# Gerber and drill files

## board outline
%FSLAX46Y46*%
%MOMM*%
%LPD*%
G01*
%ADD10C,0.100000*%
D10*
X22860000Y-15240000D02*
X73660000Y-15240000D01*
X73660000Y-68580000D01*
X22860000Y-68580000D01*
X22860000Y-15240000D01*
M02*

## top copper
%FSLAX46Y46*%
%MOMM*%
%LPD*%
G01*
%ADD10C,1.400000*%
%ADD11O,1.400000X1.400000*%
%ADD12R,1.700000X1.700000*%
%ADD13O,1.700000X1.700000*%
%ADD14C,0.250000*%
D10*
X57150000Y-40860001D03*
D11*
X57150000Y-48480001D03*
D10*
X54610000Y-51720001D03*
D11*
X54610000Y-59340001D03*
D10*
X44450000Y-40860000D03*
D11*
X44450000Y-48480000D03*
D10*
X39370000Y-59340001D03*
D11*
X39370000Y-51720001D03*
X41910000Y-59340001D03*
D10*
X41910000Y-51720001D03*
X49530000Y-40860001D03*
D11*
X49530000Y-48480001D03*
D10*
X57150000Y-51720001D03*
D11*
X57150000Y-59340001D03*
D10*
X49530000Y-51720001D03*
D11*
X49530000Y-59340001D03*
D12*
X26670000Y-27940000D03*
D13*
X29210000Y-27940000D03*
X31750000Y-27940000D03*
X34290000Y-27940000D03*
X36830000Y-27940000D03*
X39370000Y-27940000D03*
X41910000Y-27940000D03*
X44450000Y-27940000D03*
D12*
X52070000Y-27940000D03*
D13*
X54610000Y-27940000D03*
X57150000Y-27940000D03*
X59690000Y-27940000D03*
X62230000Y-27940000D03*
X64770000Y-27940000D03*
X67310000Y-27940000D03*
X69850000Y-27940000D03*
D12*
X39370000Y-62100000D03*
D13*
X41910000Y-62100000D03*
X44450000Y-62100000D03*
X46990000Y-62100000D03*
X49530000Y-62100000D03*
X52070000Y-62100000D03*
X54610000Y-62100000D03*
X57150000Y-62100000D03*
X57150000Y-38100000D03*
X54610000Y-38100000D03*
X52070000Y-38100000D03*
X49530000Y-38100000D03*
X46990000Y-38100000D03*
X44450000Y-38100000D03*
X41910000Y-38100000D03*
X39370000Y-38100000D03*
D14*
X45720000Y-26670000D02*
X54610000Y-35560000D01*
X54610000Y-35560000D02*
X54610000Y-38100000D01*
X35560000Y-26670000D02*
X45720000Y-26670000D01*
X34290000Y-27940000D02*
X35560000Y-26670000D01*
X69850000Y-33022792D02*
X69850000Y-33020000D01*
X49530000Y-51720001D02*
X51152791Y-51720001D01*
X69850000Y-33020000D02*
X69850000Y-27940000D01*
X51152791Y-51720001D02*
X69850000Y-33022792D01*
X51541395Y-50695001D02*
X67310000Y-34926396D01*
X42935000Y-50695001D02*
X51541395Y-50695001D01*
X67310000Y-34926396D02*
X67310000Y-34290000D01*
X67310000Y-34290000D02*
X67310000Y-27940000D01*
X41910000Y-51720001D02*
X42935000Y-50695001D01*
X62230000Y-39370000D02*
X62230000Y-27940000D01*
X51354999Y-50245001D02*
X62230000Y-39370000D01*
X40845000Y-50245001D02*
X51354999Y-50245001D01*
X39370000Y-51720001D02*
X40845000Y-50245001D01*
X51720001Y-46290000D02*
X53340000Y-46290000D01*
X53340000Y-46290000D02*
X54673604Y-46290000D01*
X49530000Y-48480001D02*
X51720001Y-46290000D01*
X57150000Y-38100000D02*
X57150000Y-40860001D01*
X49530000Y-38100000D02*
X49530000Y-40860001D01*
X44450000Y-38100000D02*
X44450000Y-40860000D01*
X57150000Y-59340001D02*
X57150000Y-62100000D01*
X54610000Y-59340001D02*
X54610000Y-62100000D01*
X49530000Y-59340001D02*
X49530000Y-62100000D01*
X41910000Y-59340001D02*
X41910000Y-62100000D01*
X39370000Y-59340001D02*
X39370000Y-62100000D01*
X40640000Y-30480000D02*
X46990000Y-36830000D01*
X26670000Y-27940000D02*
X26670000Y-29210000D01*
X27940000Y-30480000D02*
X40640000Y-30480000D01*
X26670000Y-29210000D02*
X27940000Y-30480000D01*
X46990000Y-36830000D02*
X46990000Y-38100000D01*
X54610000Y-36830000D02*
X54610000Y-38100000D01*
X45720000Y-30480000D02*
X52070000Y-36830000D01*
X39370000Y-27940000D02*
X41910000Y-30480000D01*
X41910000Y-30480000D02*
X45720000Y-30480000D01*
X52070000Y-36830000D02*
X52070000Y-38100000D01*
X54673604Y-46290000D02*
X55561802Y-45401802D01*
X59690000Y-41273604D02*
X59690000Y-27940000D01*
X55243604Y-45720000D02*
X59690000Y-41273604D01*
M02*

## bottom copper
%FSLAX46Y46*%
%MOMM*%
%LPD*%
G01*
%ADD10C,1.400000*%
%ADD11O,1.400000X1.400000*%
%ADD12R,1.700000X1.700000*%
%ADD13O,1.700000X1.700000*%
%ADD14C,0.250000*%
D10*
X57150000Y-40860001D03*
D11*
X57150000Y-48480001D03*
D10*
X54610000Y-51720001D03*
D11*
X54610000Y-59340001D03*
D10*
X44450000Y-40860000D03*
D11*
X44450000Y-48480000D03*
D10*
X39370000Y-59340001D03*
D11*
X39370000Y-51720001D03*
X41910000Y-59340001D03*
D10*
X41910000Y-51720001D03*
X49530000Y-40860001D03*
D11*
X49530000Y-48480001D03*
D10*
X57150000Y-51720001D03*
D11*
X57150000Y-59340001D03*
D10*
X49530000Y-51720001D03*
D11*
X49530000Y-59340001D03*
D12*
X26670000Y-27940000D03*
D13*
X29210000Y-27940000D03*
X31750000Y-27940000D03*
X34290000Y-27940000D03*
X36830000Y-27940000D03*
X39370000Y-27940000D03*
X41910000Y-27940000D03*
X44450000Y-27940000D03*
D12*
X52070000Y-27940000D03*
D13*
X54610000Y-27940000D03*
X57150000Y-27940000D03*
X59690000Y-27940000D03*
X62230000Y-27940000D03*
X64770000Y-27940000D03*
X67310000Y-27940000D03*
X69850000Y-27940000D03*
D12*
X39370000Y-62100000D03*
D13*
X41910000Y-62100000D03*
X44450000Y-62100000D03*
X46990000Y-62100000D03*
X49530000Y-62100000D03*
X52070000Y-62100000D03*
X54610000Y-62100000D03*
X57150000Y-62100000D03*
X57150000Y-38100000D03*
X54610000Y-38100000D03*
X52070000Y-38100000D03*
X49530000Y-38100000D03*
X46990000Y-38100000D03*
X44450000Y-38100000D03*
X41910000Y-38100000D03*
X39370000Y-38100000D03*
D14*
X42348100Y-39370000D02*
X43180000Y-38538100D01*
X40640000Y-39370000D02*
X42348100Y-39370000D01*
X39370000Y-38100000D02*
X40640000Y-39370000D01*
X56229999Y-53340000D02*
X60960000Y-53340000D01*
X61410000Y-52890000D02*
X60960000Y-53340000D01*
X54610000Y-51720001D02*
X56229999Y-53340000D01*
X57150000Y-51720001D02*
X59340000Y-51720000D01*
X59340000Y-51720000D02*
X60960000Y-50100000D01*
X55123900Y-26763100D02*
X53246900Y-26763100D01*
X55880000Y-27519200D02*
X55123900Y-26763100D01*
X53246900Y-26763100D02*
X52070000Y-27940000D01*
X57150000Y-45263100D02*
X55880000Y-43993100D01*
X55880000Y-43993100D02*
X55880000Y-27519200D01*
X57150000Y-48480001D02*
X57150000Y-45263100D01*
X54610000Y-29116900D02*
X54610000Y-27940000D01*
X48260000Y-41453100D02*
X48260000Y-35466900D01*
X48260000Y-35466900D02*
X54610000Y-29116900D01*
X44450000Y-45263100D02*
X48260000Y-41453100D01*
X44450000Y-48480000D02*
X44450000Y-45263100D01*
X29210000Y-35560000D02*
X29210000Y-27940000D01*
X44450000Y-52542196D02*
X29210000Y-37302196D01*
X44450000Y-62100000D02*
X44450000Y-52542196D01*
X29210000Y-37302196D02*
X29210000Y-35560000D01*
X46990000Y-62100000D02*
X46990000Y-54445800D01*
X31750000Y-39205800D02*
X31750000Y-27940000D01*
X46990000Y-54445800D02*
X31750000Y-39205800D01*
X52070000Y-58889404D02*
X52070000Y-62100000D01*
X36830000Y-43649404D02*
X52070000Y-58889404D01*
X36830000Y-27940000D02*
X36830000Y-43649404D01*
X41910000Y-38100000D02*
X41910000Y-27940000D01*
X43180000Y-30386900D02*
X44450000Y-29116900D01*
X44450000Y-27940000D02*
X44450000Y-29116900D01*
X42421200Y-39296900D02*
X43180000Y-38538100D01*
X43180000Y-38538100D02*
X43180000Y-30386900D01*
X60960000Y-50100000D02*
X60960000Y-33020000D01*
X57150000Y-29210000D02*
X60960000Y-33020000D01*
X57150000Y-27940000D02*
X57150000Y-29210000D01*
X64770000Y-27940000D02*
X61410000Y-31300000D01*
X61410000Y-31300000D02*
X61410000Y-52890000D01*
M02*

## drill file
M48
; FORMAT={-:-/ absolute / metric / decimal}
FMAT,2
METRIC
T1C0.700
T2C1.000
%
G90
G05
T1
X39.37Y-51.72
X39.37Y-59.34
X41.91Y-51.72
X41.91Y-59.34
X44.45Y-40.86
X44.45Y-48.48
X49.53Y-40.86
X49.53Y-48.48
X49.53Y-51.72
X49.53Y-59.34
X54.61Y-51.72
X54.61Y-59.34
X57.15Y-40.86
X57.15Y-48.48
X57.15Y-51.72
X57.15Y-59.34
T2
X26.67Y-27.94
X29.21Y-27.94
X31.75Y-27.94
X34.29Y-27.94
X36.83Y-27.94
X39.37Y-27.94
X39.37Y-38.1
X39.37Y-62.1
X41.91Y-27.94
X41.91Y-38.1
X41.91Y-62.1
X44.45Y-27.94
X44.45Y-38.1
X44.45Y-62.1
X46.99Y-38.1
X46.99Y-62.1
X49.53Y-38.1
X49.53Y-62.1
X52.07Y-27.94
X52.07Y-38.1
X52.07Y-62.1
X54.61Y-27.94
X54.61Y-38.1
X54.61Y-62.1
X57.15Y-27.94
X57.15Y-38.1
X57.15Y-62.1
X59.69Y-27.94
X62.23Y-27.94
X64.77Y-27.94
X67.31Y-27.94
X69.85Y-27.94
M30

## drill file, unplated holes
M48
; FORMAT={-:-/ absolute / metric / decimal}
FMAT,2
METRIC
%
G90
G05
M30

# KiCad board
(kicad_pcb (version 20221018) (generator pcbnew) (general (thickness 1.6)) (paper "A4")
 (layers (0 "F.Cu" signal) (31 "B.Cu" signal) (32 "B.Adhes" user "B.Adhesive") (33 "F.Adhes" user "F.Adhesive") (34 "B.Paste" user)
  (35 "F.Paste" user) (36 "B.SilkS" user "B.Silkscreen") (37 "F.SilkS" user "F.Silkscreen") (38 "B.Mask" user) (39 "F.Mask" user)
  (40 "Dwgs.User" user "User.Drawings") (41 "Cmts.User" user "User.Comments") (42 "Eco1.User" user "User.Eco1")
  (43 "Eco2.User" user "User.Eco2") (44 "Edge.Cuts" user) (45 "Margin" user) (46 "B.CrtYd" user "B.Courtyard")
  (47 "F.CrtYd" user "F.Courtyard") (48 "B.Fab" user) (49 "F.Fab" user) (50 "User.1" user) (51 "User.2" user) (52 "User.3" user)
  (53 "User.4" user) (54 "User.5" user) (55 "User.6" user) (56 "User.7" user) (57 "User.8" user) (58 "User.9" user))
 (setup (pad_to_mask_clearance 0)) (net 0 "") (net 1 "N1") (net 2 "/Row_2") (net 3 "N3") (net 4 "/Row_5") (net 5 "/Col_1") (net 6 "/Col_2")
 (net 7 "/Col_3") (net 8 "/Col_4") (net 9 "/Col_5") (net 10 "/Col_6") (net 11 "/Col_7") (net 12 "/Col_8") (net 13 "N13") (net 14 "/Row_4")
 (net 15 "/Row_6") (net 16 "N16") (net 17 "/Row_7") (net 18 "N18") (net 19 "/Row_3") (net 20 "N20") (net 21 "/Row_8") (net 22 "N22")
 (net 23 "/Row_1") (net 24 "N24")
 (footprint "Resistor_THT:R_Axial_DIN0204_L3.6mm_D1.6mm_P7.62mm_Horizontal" (layer "F.Cu") (at 44.45 40.86 -90)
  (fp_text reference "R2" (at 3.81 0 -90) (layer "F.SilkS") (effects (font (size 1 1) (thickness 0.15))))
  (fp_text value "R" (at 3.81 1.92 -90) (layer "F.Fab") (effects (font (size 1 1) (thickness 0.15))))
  (pad "1" thru_hole circle (at 0 0 270) (size 1.4 1.4) (drill 0.7) (layers "*.Cu" "*.Mask") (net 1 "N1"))
  (pad "2" thru_hole oval (at 7.62 0 270) (size 1.4 1.4) (drill 0.7) (layers "*.Cu" "*.Mask") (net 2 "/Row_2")))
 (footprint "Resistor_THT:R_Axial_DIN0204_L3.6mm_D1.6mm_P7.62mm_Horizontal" (layer "F.Cu") (at 39.37 59.340001 90)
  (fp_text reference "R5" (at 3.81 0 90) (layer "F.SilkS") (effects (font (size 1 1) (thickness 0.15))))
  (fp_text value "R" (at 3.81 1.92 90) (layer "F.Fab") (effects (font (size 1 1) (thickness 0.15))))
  (pad "1" thru_hole circle (at 0 0 90) (size 1.4 1.4) (drill 0.7) (layers "*.Cu" "*.Mask") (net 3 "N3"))
  (pad "2" thru_hole oval (at 7.62 0 90) (size 1.4 1.4) (drill 0.7) (layers "*.Cu" "*.Mask") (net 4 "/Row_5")))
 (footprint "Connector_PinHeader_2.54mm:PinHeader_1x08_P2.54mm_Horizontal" (layer "F.Cu") (at 26.67 27.94 90)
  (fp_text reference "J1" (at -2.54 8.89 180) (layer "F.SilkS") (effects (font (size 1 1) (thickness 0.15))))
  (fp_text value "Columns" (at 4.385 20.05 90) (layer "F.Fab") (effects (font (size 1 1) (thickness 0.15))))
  (pad "1" thru_hole rect (at 0 0 90) (size 1.7 1.7) (drill 1) (layers "*.Cu" "*.Mask") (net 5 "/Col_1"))
  (pad "2" thru_hole oval (at 0 2.54 90) (size 1.7 1.7) (drill 1) (layers "*.Cu" "*.Mask") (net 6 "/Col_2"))
  (pad "3" thru_hole oval (at 0 5.08 90) (size 1.7 1.7) (drill 1) (layers "*.Cu" "*.Mask") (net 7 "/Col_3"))
  (pad "4" thru_hole oval (at 0 7.62 90) (size 1.7 1.7) (drill 1) (layers "*.Cu" "*.Mask") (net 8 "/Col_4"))
  (pad "5" thru_hole oval (at 0 10.16 90) (size 1.7 1.7) (drill 1) (layers "*.Cu" "*.Mask") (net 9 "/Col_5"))
  (pad "6" thru_hole oval (at 0 12.7 90) (size 1.7 1.7) (drill 1) (layers "*.Cu" "*.Mask") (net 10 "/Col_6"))
  (pad "7" thru_hole oval (at 0 15.24 90) (size 1.7 1.7) (drill 1) (layers "*.Cu" "*.Mask") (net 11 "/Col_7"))
  (pad "8" thru_hole oval (at 0 17.78 90) (size 1.7 1.7) (drill 1) (layers "*.Cu" "*.Mask") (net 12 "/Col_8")))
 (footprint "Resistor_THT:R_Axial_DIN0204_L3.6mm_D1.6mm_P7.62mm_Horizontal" (layer "F.Cu") (at 49.53 40.860001 -90)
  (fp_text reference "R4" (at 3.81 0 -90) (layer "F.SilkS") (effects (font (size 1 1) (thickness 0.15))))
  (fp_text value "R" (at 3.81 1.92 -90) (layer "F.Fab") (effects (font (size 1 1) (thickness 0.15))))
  (pad "1" thru_hole circle (at 0 0 270) (size 1.4 1.4) (drill 0.7) (layers "*.Cu" "*.Mask") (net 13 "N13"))
  (pad "2" thru_hole oval (at 7.62 0 270) (size 1.4 1.4) (drill 0.7) (layers "*.Cu" "*.Mask") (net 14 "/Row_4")))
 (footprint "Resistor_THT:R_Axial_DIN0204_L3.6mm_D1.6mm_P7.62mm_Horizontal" (layer "F.Cu") (at 54.61 51.720001 -90)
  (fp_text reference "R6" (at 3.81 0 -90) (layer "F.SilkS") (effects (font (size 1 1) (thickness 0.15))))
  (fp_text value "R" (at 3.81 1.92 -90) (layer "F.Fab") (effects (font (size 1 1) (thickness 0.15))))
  (pad "1" thru_hole circle (at 0 0 270) (size 1.4 1.4) (drill 0.7) (layers "*.Cu" "*.Mask") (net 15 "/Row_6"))
  (pad "2" thru_hole oval (at 7.62 0 270) (size 1.4 1.4) (drill 0.7) (layers "*.Cu" "*.Mask") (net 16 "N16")))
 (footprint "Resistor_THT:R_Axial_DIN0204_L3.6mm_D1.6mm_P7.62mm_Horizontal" (layer "F.Cu") (at 41.91 51.720001 -90)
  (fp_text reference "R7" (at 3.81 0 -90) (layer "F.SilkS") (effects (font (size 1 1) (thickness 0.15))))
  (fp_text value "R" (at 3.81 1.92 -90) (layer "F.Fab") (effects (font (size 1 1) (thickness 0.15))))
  (pad "1" thru_hole circle (at 0 0 270) (size 1.4 1.4) (drill 0.7) (layers "*.Cu" "*.Mask") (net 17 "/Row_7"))
  (pad "2" thru_hole oval (at 7.62 0 270) (size 1.4 1.4) (drill 0.7) (layers "*.Cu" "*.Mask") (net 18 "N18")))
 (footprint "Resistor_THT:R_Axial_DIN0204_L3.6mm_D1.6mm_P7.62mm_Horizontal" (layer "F.Cu") (at 57.15 51.720001 -90)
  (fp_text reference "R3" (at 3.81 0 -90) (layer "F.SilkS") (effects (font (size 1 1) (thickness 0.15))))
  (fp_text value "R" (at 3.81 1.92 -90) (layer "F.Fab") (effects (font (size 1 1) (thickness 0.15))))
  (pad "1" thru_hole circle (at 0 0 270) (size 1.4 1.4) (drill 0.7) (layers "*.Cu" "*.Mask") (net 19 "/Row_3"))
  (pad "2" thru_hole oval (at 7.62 0 270) (size 1.4 1.4) (drill 0.7) (layers "*.Cu" "*.Mask") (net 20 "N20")))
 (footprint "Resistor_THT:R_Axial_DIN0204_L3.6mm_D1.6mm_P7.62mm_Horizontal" (layer "F.Cu") (at 49.53 51.720001 -90)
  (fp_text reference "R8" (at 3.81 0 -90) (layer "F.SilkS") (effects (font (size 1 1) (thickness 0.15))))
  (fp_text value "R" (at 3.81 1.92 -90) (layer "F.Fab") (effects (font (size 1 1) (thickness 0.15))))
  (pad "1" thru_hole circle (at 0 0 270) (size 1.4 1.4) (drill 0.7) (layers "*.Cu" "*.Mask") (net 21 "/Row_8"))
  (pad "2" thru_hole oval (at 7.62 0 270) (size 1.4 1.4) (drill 0.7) (layers "*.Cu" "*.Mask") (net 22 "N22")))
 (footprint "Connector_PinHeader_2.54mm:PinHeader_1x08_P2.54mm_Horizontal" (layer "F.Cu") (at 52.07 27.94 90)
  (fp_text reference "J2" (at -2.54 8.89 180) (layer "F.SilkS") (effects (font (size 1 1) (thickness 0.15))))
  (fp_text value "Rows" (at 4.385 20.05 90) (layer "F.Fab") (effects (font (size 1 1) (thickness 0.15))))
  (pad "1" thru_hole rect (at 0 0 90) (size 1.7 1.7) (drill 1) (layers "*.Cu" "*.Mask") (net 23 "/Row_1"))
  (pad "2" thru_hole oval (at 0 2.54 90) (size 1.7 1.7) (drill 1) (layers "*.Cu" "*.Mask") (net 2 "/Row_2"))
  (pad "3" thru_hole oval (at 0 5.08 90) (size 1.7 1.7) (drill 1) (layers "*.Cu" "*.Mask") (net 19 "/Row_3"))
  (pad "4" thru_hole oval (at 0 7.62 90) (size 1.7 1.7) (drill 1) (layers "*.Cu" "*.Mask") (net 14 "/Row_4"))
  (pad "5" thru_hole oval (at 0 10.16 90) (size 1.7 1.7) (drill 1) (layers "*.Cu" "*.Mask") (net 4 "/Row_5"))
  (pad "6" thru_hole oval (at 0 12.7 90) (size 1.7 1.7) (drill 1) (layers "*.Cu" "*.Mask") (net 15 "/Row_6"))
  (pad "7" thru_hole oval (at 0 15.24 90) (size 1.7 1.7) (drill 1) (layers "*.Cu" "*.Mask") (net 17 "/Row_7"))
  (pad "8" thru_hole oval (at 0 17.78 90) (size 1.7 1.7) (drill 1) (layers "*.Cu" "*.Mask") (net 21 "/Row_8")))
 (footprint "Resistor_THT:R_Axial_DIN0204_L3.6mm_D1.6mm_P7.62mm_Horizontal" (layer "F.Cu") (at 57.15 40.860001 -90)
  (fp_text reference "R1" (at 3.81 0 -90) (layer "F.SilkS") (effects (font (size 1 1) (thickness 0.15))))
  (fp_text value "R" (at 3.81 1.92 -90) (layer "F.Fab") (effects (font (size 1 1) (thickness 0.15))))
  (pad "1" thru_hole circle (at 0 0 270) (size 1.4 1.4) (drill 0.7) (layers "*.Cu" "*.Mask") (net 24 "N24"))
  (pad "2" thru_hole oval (at 7.62 0 270) (size 1.4 1.4) (drill 0.7) (layers "*.Cu" "*.Mask") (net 23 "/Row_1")))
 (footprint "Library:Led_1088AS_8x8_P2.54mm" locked (layer "F.Cu") (at 48.26 50.1)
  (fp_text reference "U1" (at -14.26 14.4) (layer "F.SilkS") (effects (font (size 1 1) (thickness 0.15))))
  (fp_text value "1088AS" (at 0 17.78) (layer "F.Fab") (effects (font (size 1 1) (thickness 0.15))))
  (pad "1" thru_hole rect locked (at -8.89 12) (size 1.7 1.7) (drill 1) (layers "*.Cu" "*.Mask") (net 3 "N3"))
  (pad "2" thru_hole oval locked (at -6.35 12) (size 1.7 1.7) (drill 1) (layers "*.Cu" "*.Mask") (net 18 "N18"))
  (pad "3" thru_hole oval locked (at -3.81 12) (size 1.7 1.7) (drill 1) (layers "*.Cu" "*.Mask") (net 6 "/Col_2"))
  (pad "4" thru_hole oval locked (at -1.27 12) (size 1.7 1.7) (drill 1) (layers "*.Cu" "*.Mask") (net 7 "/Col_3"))
  (pad "5" thru_hole oval locked (at 1.27 12) (size 1.7 1.7) (drill 1) (layers "*.Cu" "*.Mask") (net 22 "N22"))
  (pad "6" thru_hole oval locked (at 3.81 12) (size 1.7 1.7) (drill 1) (layers "*.Cu" "*.Mask") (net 9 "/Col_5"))
  (pad "7" thru_hole oval locked (at 6.35 12) (size 1.7 1.7) (drill 1) (layers "*.Cu" "*.Mask") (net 16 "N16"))
  (pad "8" thru_hole oval locked (at 8.89 12) (size 1.7 1.7) (drill 1) (layers "*.Cu" "*.Mask") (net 20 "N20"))
  (pad "9" thru_hole oval locked (at 8.89 -12) (size 1.7 1.7) (drill 1) (layers "*.Cu" "*.Mask") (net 24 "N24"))
  (pad "10" thru_hole oval locked (at 6.35 -12) (size 1.7 1.7) (drill 1) (layers "*.Cu" "*.Mask") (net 8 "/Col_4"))
  (pad "11" thru_hole oval locked (at 3.81 -12) (size 1.7 1.7) (drill 1) (layers "*.Cu" "*.Mask") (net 10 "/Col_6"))
  (pad "12" thru_hole oval locked (at 1.27 -12) (size 1.7 1.7) (drill 1) (layers "*.Cu" "*.Mask") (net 13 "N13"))
  (pad "13" thru_hole oval locked (at -1.27 -12) (size 1.7 1.7) (drill 1) (layers "*.Cu" "*.Mask") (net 5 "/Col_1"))
  (pad "14" thru_hole oval locked (at -3.81 -12) (size 1.7 1.7) (drill 1) (layers "*.Cu" "*.Mask") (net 1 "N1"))
  (pad "15" thru_hole oval locked (at -6.35 -12) (size 1.7 1.7) (drill 1) (layers "*.Cu" "*.Mask") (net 11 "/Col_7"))
  (pad "16" thru_hole oval locked (at -8.89 -12) (size 1.7 1.7) (drill 1) (layers "*.Cu" "*.Mask") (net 12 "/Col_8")))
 (gr_rect (start 22.86 15.24) (end 73.66 68.58) (stroke (width 0.1) (type default)) (fill none) (layer "Edge.Cuts"))
 (segment (start 40.64 30.48) (end 46.99 36.83) (width 0.25) (layer "F.Cu") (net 5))
 (segment (start 26.67 27.94) (end 26.67 29.21) (width 0.25) (layer "F.Cu") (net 5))
 (segment (start 27.94 30.48) (end 40.64 30.48) (width 0.25) (layer "F.Cu") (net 5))
 (segment (start 26.67 29.21) (end 27.94 30.48) (width 0.25) (layer "F.Cu") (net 5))
 (segment (start 46.99 36.83) (end 46.99 38.1) (width 0.25) (layer "F.Cu") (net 5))
 (segment (start 29.21 35.56) (end 29.21 27.94) (width 0.25) (layer "B.Cu") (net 6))
 (segment (start 44.45 52.542196) (end 29.21 37.302196) (width 0.25) (layer "B.Cu") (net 6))
 (segment (start 44.45 62.1) (end 44.45 52.542196) (width 0.25) (layer "B.Cu") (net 6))
 (segment (start 29.21 37.302196) (end 29.21 35.56) (width 0.25) (layer "B.Cu") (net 6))
 (segment (start 46.99 62.1) (end 46.99 54.4458) (width 0.25) (layer "B.Cu") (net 7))
 (segment (start 31.75 39.2058) (end 31.75 27.94) (width 0.25) (layer "B.Cu") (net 7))
 (segment (start 46.99 54.4458) (end 31.75 39.2058) (width 0.25) (layer "B.Cu") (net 7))
 (segment (start 54.61 35.56) (end 54.61 38.1) (width 0.25) (layer "F.Cu") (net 8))
 (segment (start 34.29 27.94) (end 35.56 26.67) (width 0.25) (layer "F.Cu") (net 8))
 (segment (start 35.56 26.67) (end 45.72 26.67) (width 0.25) (layer "F.Cu") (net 8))
 (segment (start 54.61 36.83) (end 54.61 38.1) (width 0.25) (layer "F.Cu") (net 8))
 (segment (start 45.72 26.67) (end 54.61 35.56) (width 0.25) (layer "F.Cu") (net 8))
 (segment (start 52.07 58.889404) (end 52.07 62.1) (width 0.25) (layer "B.Cu") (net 9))
 (segment (start 36.83 43.649404) (end 52.07 58.889404) (width 0.25) (layer "B.Cu") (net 9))
 (segment (start 36.83 27.94) (end 36.83 43.649404) (width 0.25) (layer "B.Cu") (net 9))
 (segment (start 45.72 30.48) (end 52.07 36.83) (width 0.25) (layer "F.Cu") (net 10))
 (segment (start 39.37 27.94) (end 41.91 30.48) (width 0.25) (layer "F.Cu") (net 10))
 (segment (start 41.91 30.48) (end 45.72 30.48) (width 0.25) (layer "F.Cu") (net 10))
 (segment (start 52.07 36.83) (end 52.07 38.1) (width 0.25) (layer "F.Cu") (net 10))
 (segment (start 41.91 38.1) (end 41.91 27.94) (width 0.25) (layer "B.Cu") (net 11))
 (segment (start 39.37 38.1) (end 40.64 39.37) (width 0.25) (layer "B.Cu") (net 12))
 (segment (start 43.18 30.3869) (end 44.45 29.1169) (width 0.25) (layer "B.Cu") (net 12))
 (segment (start 44.45 27.94) (end 44.45 29.1169) (width 0.25) (layer "B.Cu") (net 12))
 (segment (start 42.4212 39.2969) (end 43.18 38.5381) (width 0.25) (layer "B.Cu") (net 12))
 (segment (start 43.18 38.5381) (end 43.18 30.3869) (width 0.25) (layer "B.Cu") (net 12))
 (segment (start 40.64 39.37) (end 42.3481 39.37) (width 0.25) (layer "B.Cu") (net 12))
 (segment (start 42.3481 39.37) (end 43.18 38.5381) (width 0.25) (layer "B.Cu") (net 12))
 (segment (start 57.15 48.480001) (end 57.15 45.2631) (width 0.25) (layer "B.Cu") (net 23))
 (segment (start 55.88 43.9931) (end 55.88 27.5192) (width 0.25) (layer "B.Cu") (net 23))
 (segment (start 55.1239 26.7631) (end 53.2469 26.7631) (width 0.25) (layer "B.Cu") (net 23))
 (segment (start 57.15 45.2631) (end 55.88 43.9931) (width 0.25) (layer "B.Cu") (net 23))
 (segment (start 53.2469 26.7631) (end 52.07 27.94) (width 0.25) (layer "B.Cu") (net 23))
 (segment (start 55.88 27.5192) (end 55.1239 26.7631) (width 0.25) (layer "B.Cu") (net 23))
 (segment (start 48.26 35.4669) (end 54.61 29.1169) (width 0.25) (layer "B.Cu") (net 2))
 (segment (start 44.45 45.2631) (end 48.26 41.4531) (width 0.25) (layer "B.Cu") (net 2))
 (segment (start 48.26 41.4531) (end 48.26 35.4669) (width 0.25) (layer "B.Cu") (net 2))
 (segment (start 44.45 48.48) (end 44.45 45.2631) (width 0.25) (layer "B.Cu") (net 2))
 (segment (start 54.61 29.1169) (end 54.61 27.94) (width 0.25) (layer "B.Cu") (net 2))
 (segment (start 60.96 50.1) (end 60.96 33.02) (width 0.25) (layer "B.Cu") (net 19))
 (segment (start 57.15 29.21) (end 60.96 33.02) (width 0.25) (layer "B.Cu") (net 19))
 (segment (start 57.15 27.94) (end 57.15 29.21) (width 0.25) (layer "B.Cu") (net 19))
 (segment (start 59.34 51.72) (end 60.96 50.1) (width 0.25) (layer "B.Cu") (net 19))
 (segment (start 57.15 51.720001) (end 59.34 51.72) (width 0.25) (layer "B.Cu") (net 19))
 (segment (start 49.53 48.480001) (end 51.720001 46.29) (width 0.25) (layer "F.Cu") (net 14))
 (segment (start 54.673604 46.29) (end 55.561802 45.401802) (width 0.25) (layer "F.Cu") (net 14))
 (segment (start 59.69 41.273604) (end 59.69 27.94) (width 0.25) (layer "F.Cu") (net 14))
 (segment (start 55.243604 45.72) (end 59.69 41.273604) (width 0.25) (layer "F.Cu") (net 14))
 (segment (start 51.720001 46.29) (end 53.34 46.29) (width 0.25) (layer "F.Cu") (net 14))
 (segment (start 53.34 46.29) (end 54.673604 46.29) (width 0.25) (layer "F.Cu") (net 14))
 (segment (start 39.37 51.720001) (end 40.845 50.245001) (width 0.25) (layer "F.Cu") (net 4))
 (segment (start 51.354999 50.245001) (end 62.23 39.37) (width 0.25) (layer "F.Cu") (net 4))
 (segment (start 40.845 50.245001) (end 51.354999 50.245001) (width 0.25) (layer "F.Cu") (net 4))
 (segment (start 62.23 39.37) (end 62.23 27.94) (width 0.25) (layer "F.Cu") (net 4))
 (segment (start 64.77 27.94) (end 61.41 31.3) (width 0.25) (layer "B.Cu") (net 15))
 (segment (start 61.41 52.89) (end 60.96 53.34) (width 0.25) (layer "B.Cu") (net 15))
 (segment (start 56.229999 53.34) (end 60.96 53.34) (width 0.25) (layer "B.Cu") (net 15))
 (segment (start 54.61 51.720001) (end 56.229999 53.34) (width 0.25) (layer "B.Cu") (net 15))
 (segment (start 61.41 31.3) (end 61.41 52.89) (width 0.25) (layer "B.Cu") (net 15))
 (segment (start 42.935 50.695001) (end 51.541395 50.695001) (width 0.25) (layer "F.Cu") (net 17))
 (segment (start 41.91 51.720001) (end 42.935 50.695001) (width 0.25) (layer "F.Cu") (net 17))
 (segment (start 67.31 34.926396) (end 67.31 34.29) (width 0.25) (layer "F.Cu") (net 17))
 (segment (start 67.31 34.29) (end 67.31 27.94) (width 0.25) (layer "F.Cu") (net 17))
 (segment (start 51.541395 50.695001) (end 67.31 34.926396) (width 0.25) (layer "F.Cu") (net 17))
 (segment (start 51.152791 51.720001) (end 69.85 33.022792) (width 0.25) (layer "F.Cu") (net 21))
 (segment (start 49.53 51.720001) (end 51.152791 51.720001) (width 0.25) (layer "F.Cu") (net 21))
 (segment (start 69.85 33.022792) (end 69.85 33.02) (width 0.25) (layer "F.Cu") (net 21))
 (segment (start 69.85 33.02) (end 69.85 27.94) (width 0.25) (layer "F.Cu") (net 21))
 (segment (start 57.15 38.1) (end 57.15 40.860001) (width 0.25) (layer "F.Cu") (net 24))
 (segment (start 44.45 38.1) (end 44.45 40.86) (width 0.25) (layer "F.Cu") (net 1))
 (segment (start 57.15 59.340001) (end 57.15 62.1) (width 0.25) (layer "F.Cu") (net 20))
 (segment (start 49.53 38.1) (end 49.53 40.860001) (width 0.25) (layer "F.Cu") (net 13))
 (segment (start 39.37 59.340001) (end 39.37 62.1) (width 0.25) (layer "F.Cu") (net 3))
 (segment (start 54.61 59.340001) (end 54.61 62.1) (width 0.25) (layer "F.Cu") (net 16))
 (segment (start 41.91 59.340001) (end 41.91 62.1) (width 0.25) (layer "F.Cu") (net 18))
 (segment (start 49.53 59.340001) (end 49.53 62.1) (width 0.25) (layer "F.Cu") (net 22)))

